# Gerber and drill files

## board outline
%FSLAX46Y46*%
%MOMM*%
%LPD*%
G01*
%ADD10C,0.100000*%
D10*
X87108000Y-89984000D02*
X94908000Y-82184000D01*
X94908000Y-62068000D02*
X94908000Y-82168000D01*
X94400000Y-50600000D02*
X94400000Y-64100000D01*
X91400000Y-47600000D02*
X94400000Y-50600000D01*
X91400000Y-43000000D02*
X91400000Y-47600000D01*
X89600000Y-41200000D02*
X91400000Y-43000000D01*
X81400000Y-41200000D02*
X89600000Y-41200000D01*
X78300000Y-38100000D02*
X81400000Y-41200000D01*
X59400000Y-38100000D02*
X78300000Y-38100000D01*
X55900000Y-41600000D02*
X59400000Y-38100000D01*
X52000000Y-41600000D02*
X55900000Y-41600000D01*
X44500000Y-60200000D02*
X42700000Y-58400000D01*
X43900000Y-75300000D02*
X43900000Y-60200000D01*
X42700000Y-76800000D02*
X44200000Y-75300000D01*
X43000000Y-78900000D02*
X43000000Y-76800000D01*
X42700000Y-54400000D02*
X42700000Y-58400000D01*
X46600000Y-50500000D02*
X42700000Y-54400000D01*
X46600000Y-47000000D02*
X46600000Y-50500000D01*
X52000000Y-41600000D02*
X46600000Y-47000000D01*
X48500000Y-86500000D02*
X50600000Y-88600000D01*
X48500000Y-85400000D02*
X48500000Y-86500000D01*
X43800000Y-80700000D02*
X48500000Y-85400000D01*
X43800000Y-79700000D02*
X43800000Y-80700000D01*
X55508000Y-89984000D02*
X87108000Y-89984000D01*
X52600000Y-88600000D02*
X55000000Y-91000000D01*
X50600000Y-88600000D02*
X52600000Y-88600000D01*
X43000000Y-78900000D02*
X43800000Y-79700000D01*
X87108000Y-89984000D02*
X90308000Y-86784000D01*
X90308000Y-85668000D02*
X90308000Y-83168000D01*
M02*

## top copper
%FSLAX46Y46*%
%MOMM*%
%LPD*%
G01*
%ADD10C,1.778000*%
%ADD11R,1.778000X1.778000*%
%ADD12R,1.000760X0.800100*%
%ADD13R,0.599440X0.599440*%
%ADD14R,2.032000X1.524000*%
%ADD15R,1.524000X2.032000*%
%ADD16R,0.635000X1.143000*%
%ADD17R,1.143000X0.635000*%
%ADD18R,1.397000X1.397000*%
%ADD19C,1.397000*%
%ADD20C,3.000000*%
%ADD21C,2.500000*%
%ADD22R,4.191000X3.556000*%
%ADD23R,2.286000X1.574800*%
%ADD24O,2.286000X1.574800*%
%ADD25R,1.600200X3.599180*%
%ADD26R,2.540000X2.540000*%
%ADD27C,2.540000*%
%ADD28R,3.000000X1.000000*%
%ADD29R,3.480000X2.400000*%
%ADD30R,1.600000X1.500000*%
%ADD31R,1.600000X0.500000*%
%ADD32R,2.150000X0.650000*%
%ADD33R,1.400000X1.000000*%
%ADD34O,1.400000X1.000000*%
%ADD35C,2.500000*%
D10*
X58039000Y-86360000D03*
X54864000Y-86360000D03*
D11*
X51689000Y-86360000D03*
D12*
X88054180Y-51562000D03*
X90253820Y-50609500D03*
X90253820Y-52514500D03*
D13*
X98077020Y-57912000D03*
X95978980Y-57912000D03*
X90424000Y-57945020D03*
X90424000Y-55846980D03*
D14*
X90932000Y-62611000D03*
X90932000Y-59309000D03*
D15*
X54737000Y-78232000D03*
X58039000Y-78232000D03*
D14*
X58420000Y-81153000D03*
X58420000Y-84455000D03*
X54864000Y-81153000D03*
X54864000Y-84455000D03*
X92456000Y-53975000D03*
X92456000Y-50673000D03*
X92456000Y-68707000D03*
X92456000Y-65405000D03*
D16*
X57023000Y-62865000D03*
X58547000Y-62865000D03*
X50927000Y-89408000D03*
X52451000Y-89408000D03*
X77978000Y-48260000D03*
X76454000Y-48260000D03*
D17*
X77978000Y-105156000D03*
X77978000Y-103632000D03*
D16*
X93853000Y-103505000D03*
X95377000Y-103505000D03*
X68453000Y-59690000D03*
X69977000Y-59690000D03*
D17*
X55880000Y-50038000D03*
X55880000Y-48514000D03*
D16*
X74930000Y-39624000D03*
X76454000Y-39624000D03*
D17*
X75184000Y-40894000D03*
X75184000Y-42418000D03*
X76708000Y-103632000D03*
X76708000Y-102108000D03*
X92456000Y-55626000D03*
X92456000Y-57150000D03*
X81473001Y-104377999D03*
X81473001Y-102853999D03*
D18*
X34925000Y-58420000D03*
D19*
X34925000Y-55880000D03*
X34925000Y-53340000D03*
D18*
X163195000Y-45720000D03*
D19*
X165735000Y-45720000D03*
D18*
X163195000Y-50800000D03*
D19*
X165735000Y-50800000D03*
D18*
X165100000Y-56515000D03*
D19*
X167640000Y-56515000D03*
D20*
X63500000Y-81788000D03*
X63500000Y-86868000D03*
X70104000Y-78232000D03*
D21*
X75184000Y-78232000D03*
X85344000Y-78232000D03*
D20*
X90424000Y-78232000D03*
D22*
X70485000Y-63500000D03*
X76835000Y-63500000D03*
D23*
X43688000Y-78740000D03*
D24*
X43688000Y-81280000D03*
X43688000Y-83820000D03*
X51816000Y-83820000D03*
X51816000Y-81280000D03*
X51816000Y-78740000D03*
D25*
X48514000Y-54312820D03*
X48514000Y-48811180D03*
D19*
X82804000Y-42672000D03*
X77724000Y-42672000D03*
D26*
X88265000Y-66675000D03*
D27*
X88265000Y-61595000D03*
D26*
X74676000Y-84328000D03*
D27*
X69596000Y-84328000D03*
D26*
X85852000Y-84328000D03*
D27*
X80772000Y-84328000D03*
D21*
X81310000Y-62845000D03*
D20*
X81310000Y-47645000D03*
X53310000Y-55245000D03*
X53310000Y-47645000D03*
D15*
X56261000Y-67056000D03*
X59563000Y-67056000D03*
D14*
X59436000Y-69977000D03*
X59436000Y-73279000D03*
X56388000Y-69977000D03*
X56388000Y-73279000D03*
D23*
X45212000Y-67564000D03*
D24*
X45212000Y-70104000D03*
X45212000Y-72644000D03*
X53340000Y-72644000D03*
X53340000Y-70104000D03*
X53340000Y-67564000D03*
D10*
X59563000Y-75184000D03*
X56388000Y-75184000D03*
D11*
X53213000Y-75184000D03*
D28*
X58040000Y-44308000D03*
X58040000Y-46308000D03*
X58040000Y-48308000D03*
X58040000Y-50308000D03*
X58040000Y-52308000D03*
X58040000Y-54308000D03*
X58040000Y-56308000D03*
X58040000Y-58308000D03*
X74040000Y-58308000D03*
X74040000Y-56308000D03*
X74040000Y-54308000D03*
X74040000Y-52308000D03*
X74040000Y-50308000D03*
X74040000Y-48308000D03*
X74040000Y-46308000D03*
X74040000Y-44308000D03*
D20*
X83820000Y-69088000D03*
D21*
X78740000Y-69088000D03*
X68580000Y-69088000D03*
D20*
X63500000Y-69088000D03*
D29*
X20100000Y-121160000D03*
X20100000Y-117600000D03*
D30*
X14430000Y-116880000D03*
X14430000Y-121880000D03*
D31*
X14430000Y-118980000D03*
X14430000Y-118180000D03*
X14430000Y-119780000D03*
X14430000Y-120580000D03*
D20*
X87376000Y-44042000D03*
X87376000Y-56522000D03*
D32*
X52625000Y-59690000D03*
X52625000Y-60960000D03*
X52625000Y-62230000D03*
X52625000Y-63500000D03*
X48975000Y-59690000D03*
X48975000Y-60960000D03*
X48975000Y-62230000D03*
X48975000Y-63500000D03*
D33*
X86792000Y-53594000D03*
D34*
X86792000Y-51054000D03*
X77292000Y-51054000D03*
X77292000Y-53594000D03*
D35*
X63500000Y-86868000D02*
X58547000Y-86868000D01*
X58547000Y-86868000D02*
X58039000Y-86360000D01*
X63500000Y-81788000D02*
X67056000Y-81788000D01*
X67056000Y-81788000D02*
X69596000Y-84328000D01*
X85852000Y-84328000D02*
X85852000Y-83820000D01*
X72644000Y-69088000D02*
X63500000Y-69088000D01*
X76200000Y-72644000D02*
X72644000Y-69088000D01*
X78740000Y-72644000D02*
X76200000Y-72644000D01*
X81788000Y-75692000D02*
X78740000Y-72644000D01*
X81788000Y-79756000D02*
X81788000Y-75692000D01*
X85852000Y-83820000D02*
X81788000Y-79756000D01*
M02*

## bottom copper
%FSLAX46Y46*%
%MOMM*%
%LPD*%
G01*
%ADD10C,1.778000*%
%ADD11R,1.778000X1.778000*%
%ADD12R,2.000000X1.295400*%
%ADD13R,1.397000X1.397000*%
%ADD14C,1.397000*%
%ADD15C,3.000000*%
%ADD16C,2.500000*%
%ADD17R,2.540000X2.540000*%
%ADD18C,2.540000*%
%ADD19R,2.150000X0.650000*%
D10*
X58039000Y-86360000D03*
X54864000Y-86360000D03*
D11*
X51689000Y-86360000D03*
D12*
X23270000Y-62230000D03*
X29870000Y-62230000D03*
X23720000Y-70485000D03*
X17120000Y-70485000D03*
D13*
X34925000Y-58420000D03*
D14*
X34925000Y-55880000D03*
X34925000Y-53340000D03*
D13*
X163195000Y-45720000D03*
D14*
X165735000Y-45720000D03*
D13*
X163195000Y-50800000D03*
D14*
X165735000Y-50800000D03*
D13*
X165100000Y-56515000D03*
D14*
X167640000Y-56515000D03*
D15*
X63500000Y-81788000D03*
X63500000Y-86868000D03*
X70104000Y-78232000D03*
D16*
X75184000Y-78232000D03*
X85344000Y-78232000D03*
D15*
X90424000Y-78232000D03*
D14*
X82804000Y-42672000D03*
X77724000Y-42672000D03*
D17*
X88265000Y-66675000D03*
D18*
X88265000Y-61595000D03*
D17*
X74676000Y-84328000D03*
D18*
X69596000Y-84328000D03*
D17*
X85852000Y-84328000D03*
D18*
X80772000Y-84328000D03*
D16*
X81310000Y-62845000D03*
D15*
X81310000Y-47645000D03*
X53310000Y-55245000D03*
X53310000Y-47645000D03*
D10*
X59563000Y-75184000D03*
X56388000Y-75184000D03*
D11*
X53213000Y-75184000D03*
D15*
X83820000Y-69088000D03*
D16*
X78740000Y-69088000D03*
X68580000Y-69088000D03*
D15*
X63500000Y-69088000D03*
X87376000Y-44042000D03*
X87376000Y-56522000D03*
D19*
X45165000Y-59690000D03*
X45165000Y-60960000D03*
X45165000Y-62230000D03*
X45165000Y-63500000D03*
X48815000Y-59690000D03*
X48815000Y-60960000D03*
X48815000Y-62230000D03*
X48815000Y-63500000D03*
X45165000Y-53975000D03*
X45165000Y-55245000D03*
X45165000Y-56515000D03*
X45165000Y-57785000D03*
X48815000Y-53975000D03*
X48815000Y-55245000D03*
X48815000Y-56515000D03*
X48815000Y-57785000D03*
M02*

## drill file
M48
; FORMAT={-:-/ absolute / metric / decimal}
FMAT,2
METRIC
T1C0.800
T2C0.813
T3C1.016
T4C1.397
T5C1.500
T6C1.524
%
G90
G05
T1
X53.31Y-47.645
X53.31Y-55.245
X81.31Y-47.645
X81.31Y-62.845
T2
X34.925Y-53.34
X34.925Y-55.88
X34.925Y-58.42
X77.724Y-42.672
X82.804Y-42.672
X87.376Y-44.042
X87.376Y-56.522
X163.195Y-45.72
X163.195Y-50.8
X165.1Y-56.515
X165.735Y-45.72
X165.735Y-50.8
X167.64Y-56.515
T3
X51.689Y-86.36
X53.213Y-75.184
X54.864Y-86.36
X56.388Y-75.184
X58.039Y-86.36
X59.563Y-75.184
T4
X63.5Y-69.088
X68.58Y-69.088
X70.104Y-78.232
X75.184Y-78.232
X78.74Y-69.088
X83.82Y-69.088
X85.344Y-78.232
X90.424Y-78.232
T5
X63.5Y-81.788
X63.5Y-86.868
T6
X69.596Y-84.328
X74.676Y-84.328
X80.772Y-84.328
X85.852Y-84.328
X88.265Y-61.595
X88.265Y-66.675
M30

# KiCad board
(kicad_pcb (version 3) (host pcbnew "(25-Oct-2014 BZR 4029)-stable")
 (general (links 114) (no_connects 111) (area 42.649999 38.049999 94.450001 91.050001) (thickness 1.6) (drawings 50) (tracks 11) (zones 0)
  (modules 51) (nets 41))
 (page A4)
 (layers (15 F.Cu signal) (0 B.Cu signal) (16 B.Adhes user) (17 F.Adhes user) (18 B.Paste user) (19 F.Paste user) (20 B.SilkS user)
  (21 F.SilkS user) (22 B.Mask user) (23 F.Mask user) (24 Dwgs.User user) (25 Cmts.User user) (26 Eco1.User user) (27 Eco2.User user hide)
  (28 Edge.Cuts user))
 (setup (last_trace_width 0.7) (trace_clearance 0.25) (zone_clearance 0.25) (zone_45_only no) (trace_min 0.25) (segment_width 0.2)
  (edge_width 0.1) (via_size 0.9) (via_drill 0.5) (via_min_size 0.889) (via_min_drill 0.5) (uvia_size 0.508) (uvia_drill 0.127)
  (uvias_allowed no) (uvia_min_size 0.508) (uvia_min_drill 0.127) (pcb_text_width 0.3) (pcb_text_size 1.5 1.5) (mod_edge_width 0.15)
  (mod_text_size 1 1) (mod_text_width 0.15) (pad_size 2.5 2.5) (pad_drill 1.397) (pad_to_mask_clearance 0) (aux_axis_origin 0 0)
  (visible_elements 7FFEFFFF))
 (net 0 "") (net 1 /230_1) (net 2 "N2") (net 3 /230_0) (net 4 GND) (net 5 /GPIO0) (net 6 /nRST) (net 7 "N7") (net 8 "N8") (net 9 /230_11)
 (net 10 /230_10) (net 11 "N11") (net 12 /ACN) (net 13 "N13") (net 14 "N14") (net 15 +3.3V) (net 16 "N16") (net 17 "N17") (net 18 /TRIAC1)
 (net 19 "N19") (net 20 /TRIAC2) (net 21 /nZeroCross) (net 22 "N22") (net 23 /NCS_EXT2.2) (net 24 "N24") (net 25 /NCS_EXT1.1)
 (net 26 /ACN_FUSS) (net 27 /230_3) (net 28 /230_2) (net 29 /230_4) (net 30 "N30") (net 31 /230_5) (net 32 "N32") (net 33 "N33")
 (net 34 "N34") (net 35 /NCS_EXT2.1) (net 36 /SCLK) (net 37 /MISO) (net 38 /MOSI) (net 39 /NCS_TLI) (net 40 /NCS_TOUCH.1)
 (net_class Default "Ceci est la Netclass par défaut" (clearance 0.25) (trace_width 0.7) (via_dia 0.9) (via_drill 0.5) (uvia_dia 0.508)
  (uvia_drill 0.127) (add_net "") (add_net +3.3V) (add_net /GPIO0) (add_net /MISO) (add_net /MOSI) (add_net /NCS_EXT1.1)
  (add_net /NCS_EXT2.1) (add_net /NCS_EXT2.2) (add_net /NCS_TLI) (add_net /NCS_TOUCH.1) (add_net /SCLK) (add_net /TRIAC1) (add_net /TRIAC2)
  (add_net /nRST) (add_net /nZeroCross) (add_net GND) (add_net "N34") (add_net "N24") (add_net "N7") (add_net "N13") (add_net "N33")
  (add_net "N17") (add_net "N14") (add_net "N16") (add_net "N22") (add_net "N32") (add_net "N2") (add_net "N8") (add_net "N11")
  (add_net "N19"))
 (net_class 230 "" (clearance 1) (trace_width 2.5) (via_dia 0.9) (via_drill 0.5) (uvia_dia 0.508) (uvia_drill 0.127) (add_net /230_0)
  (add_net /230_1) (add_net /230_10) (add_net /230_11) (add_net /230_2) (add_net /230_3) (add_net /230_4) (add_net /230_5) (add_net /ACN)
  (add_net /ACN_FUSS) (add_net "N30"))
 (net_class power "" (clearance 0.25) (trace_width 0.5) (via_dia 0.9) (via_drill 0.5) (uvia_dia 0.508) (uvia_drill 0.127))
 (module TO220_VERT (layer B.Cu) (at 54.864 86.36 90)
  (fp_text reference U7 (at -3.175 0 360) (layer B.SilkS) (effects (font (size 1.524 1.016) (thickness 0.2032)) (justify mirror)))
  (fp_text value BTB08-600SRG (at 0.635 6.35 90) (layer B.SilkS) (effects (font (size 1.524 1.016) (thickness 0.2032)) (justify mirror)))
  (pad 2 thru_hole circle (at 0 3.175 90) (size 1.778 1.778) (drill 1.016) (layers *.Cu *.Mask B.SilkS) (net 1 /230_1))
  (pad 3 thru_hole circle (at 0 0 90) (size 1.778 1.778) (drill 1.016) (layers *.Cu *.Mask B.SilkS) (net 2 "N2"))
  (pad 1 thru_hole rect (at 0 -3.175 90) (size 1.778 1.778) (drill 1.016) (layers *.Cu *.Mask B.SilkS) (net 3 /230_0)))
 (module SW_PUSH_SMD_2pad (layer B.Cu) (at 26.67 62.23)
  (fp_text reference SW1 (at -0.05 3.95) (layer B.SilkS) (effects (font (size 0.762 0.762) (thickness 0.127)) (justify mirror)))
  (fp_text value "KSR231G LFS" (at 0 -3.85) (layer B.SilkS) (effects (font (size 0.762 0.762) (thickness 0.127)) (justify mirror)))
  (pad 1 smd rect (at -3.4 0) (size 2 1.2954) (layers B.Cu B.Paste B.Mask) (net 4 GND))
  (pad 2 smd rect (at 3.2 0) (size 2 1.2954) (layers B.Cu B.Paste B.Mask) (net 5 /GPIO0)))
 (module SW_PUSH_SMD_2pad (layer B.Cu) (at 20.32 70.485 180)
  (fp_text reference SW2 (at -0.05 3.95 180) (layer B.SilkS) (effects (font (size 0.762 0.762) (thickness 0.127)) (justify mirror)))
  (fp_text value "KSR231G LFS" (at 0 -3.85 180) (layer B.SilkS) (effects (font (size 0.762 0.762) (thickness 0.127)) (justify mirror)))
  (pad 1 smd rect (at -3.4 0 180) (size 2 1.2954) (layers B.Cu B.Paste B.Mask) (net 4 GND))
  (pad 2 smd rect (at 3.2 0 180) (size 2 1.2954) (layers B.Cu B.Paste B.Mask) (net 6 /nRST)))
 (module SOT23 (layer F.Cu) (at 89.154 51.562 90)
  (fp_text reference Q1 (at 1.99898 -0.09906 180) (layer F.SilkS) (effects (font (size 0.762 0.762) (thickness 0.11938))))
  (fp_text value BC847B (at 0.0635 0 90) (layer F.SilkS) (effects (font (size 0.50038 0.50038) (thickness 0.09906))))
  (pad 3 smd rect (at 0 -1.09982 90) (size 0.8001 1.00076) (layers F.Cu F.Paste F.Mask) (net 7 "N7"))
  (pad 2 smd rect (at 0.9525 1.09982 90) (size 0.8001 1.00076) (layers F.Cu F.Paste F.Mask) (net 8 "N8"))
  (pad 1 smd rect (at -0.9525 1.09982 90) (size 0.8001 1.00076) (layers F.Cu F.Paste F.Mask) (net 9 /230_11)))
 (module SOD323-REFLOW (layer F.Cu) (at 97.028 57.912 180)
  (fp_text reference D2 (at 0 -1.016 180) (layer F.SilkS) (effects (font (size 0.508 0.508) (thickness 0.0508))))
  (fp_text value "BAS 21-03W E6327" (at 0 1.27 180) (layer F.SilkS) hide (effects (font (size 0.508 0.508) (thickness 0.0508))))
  (pad 1 smd rect (at -1.04902 0 180) (size 0.59944 0.59944) (layers F.Cu F.Paste F.Mask) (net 8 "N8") (clearance 0.09906))
  (pad 2 smd rect (at 1.04902 0 180) (size 0.59944 0.59944) (layers F.Cu F.Paste F.Mask) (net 9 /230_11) (clearance 0.09906)))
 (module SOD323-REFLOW (layer F.Cu) (at 90.424 56.896 90)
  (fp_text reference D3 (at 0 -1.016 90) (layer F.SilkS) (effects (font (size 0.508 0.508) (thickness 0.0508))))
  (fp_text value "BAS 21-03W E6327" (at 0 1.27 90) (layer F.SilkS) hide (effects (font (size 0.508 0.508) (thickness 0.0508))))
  (pad 1 smd rect (at -1.04902 0 90) (size 0.59944 0.59944) (layers F.Cu F.Paste F.Mask) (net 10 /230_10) (clearance 0.09906))
  (pad 2 smd rect (at 1.04902 0 90) (size 0.59944 0.59944) (layers F.Cu F.Paste F.Mask) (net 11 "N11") (clearance 0.09906)))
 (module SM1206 (layer F.Cu) (at 90.932 60.96 90)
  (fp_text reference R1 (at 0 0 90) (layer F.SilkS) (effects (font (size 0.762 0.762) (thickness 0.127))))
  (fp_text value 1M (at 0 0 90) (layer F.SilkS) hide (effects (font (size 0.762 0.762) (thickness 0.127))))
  (pad 1 smd rect (at -1.651 0 90) (size 1.524 2.032) (layers F.Cu F.Paste F.Mask) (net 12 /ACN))
  (pad 2 smd rect (at 1.651 0 90) (size 1.524 2.032) (layers F.Cu F.Paste F.Mask) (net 10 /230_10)))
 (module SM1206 (layer F.Cu) (at 56.388 78.232)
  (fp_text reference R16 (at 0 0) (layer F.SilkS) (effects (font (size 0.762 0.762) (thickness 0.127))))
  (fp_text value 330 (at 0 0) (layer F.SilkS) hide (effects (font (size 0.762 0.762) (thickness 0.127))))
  (pad 1 smd rect (at -1.651 0) (size 1.524 2.032) (layers F.Cu F.Paste F.Mask) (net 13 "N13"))
  (pad 2 smd rect (at 1.651 0) (size 1.524 2.032) (layers F.Cu F.Paste F.Mask) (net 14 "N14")))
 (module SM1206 (layer F.Cu) (at 58.42 82.804 270)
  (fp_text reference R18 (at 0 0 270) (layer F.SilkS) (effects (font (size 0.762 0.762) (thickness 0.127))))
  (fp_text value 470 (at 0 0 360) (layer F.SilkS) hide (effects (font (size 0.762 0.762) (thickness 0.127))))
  (pad 1 smd rect (at -1.651 0 270) (size 1.524 2.032) (layers F.Cu F.Paste F.Mask) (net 14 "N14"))
  (pad 2 smd rect (at 1.651 0 270) (size 1.524 2.032) (layers F.Cu F.Paste F.Mask) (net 1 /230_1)))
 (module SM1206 (layer F.Cu) (at 54.864 82.804 270)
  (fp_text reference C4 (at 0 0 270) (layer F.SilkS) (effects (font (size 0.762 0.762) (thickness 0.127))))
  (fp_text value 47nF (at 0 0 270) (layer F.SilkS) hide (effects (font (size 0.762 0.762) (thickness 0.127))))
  (pad 1 smd rect (at -1.651 0 270) (size 1.524 2.032) (layers F.Cu F.Paste F.Mask) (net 14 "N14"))
  (pad 2 smd rect (at 1.651 0 270) (size 1.524 2.032) (layers F.Cu F.Paste F.Mask) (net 2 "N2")))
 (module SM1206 (layer F.Cu) (at 92.456 52.324 90)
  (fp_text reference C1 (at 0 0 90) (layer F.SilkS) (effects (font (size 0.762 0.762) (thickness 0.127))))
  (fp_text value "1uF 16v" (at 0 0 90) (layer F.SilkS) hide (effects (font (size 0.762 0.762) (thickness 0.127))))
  (pad 1 smd rect (at -1.651 0 90) (size 1.524 2.032) (layers F.Cu F.Paste F.Mask) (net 11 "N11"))
  (pad 2 smd rect (at 1.651 0 90) (size 1.524 2.032) (layers F.Cu F.Paste F.Mask) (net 8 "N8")))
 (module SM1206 (layer F.Cu) (at 92.456 67.056 90)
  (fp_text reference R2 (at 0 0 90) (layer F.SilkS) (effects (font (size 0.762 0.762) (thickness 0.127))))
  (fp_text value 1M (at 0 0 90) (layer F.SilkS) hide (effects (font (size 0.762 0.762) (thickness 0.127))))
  (pad 1 smd rect (at -1.651 0 90) (size 1.524 2.032) (layers F.Cu F.Paste F.Mask) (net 3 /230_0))
  (pad 2 smd rect (at 1.651 0 90) (size 1.524 2.032) (layers F.Cu F.Paste F.Mask) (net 9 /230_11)))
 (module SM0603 (layer F.Cu) (at 57.785 62.865)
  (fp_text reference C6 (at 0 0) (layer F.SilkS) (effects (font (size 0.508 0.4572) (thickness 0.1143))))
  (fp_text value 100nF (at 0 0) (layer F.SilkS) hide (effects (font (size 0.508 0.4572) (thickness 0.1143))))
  (pad 1 smd rect (at -0.762 0) (size 0.635 1.143) (layers F.Cu F.Paste F.Mask) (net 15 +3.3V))
  (pad 2 smd rect (at 0.762 0) (size 0.635 1.143) (layers F.Cu F.Paste F.Mask) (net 4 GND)))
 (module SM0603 (layer F.Cu) (at 51.689 89.408)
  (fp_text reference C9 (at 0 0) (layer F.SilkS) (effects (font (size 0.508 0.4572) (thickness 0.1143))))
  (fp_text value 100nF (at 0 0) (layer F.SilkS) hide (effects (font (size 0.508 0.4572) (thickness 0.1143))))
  (pad 1 smd rect (at -0.762 0) (size 0.635 1.143) (layers F.Cu F.Paste F.Mask) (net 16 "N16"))
  (pad 2 smd rect (at 0.762 0) (size 0.635 1.143) (layers F.Cu F.Paste F.Mask) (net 4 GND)))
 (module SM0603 (layer F.Cu) (at 77.216 48.26 180)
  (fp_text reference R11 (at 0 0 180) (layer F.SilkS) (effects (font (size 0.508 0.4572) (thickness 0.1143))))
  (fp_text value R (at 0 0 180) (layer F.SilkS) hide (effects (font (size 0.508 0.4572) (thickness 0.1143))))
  (pad 1 smd rect (at -0.762 0 180) (size 0.635 1.143) (layers F.Cu F.Paste F.Mask) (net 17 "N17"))
  (pad 2 smd rect (at 0.762 0 180) (size 0.635 1.143) (layers F.Cu F.Paste F.Mask) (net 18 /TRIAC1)))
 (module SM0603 (layer F.Cu) (at 77.978 104.394 90)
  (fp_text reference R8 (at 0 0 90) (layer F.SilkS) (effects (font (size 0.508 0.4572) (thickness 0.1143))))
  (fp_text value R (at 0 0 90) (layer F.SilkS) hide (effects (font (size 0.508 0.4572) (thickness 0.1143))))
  (pad 1 smd rect (at -0.762 0 90) (size 0.635 1.143) (layers F.Cu F.Paste F.Mask) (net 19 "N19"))
  (pad 2 smd rect (at 0.762 0 90) (size 0.635 1.143) (layers F.Cu F.Paste F.Mask) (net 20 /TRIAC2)))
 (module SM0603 (layer F.Cu) (at 94.615 103.505)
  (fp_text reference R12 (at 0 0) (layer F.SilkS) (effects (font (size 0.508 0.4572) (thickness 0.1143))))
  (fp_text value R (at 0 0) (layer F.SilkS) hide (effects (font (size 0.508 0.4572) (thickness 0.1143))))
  (pad 1 smd rect (at -0.762 0) (size 0.635 1.143) (layers F.Cu F.Paste F.Mask) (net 15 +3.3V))
  (pad 2 smd rect (at 0.762 0) (size 0.635 1.143) (layers F.Cu F.Paste F.Mask) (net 16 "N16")))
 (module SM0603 (layer F.Cu) (at 69.215 59.69)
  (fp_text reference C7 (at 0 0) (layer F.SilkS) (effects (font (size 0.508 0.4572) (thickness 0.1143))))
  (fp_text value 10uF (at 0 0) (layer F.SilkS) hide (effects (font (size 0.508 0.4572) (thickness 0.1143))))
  (pad 1 smd rect (at -0.762 0) (size 0.635 1.143) (layers F.Cu F.Paste F.Mask) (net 16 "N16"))
  (pad 2 smd rect (at 0.762 0) (size 0.635 1.143) (layers F.Cu F.Paste F.Mask) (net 4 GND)))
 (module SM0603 (layer F.Cu) (at 55.88 49.276 90)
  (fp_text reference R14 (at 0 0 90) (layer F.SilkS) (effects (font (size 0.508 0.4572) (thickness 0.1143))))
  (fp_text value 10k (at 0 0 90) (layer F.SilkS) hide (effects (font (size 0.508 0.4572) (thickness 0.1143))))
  (pad 1 smd rect (at -0.762 0 90) (size 0.635 1.143) (layers F.Cu F.Paste F.Mask) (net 15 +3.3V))
  (pad 2 smd rect (at 0.762 0 90) (size 0.635 1.143) (layers F.Cu F.Paste F.Mask) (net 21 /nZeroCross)))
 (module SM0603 (layer F.Cu) (at 75.692 39.624)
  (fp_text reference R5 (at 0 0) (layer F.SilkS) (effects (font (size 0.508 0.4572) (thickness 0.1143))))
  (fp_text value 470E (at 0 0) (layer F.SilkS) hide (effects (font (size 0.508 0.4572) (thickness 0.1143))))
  (pad 1 smd rect (at -0.762 0) (size 0.635 1.143) (layers F.Cu F.Paste F.Mask) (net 15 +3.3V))
  (pad 2 smd rect (at 0.762 0) (size 0.635 1.143) (layers F.Cu F.Paste F.Mask) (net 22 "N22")))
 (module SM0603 (layer F.Cu) (at 75.184 41.656 270)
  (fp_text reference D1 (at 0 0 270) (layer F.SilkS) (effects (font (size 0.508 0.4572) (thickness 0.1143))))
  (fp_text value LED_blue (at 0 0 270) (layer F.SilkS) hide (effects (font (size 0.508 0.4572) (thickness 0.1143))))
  (pad 1 smd rect (at -0.762 0 270) (size 0.635 1.143) (layers F.Cu F.Paste F.Mask) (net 22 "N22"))
  (pad 2 smd rect (at 0.762 0 270) (size 0.635 1.143) (layers F.Cu F.Paste F.Mask) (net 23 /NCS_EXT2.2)))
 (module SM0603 (layer F.Cu) (at 76.708 102.87 90)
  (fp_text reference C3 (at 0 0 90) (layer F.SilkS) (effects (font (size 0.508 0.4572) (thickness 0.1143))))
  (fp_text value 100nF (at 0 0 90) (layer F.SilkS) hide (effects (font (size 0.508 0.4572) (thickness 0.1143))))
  (pad 1 smd rect (at -0.762 0 90) (size 0.635 1.143) (layers F.Cu F.Paste F.Mask) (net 15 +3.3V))
  (pad 2 smd rect (at 0.762 0 90) (size 0.635 1.143) (layers F.Cu F.Paste F.Mask) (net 4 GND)))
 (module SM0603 (layer F.Cu) (at 92.456 56.388 270)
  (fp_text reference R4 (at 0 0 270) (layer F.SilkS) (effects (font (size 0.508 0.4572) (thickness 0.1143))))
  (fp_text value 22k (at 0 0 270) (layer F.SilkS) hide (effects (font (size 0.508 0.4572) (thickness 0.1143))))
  (pad 1 smd rect (at -0.762 0 270) (size 0.635 1.143) (layers F.Cu F.Paste F.Mask) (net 11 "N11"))
  (pad 2 smd rect (at 0.762 0 270) (size 0.635 1.143) (layers F.Cu F.Paste F.Mask) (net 9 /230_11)))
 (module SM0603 (layer F.Cu) (at 81.473001 103.615999 90)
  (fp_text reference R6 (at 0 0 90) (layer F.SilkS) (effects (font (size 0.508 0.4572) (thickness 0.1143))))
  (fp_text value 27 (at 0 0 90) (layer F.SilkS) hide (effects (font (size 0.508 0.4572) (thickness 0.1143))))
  (pad 1 smd rect (at -0.762 0 90) (size 0.635 1.143) (layers F.Cu F.Paste F.Mask) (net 11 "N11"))
  (pad 2 smd rect (at 0.762 0 90) (size 0.635 1.143) (layers F.Cu F.Paste F.Mask) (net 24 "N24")))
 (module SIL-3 (layer F.Cu) (at 34.925 55.88 90)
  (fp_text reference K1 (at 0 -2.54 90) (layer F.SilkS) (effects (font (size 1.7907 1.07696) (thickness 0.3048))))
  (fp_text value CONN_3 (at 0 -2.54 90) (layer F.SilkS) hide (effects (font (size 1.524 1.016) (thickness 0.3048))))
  (pad 1 thru_hole rect (at -2.54 0 90) (size 1.397 1.397) (drill 0.8128) (layers *.Cu *.Mask F.SilkS) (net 4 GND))
  (pad 2 thru_hole circle (at 0 0 90) (size 1.397 1.397) (drill 0.8128) (layers *.Cu *.Mask F.SilkS) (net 23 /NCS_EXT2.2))
  (pad 3 thru_hole circle (at 2.54 0 90) (size 1.397 1.397) (drill 0.8128) (layers *.Cu *.Mask F.SilkS) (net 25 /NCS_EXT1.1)))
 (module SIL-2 (layer F.Cu) (at 164.465 45.72)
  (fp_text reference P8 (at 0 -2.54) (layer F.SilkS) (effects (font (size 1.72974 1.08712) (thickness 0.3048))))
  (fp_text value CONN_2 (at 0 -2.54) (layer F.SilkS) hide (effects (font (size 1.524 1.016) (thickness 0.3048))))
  (pad 1 thru_hole rect (at -1.27 0) (size 1.397 1.397) (drill 0.8128) (layers *.Cu *.Mask F.SilkS) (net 4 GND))
  (pad 2 thru_hole circle (at 1.27 0) (size 1.397 1.397) (drill 0.8128) (layers *.Cu *.Mask F.SilkS) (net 4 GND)))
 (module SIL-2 (layer F.Cu) (at 164.465 50.8)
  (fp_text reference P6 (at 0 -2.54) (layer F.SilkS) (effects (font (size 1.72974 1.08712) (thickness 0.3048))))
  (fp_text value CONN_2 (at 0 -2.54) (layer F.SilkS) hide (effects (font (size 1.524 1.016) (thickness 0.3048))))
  (pad 1 thru_hole rect (at -1.27 0) (size 1.397 1.397) (drill 0.8128) (layers *.Cu *.Mask F.SilkS) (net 4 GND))
  (pad 2 thru_hole circle (at 1.27 0) (size 1.397 1.397) (drill 0.8128) (layers *.Cu *.Mask F.SilkS) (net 4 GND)))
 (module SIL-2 (layer F.Cu) (at 166.37 56.515)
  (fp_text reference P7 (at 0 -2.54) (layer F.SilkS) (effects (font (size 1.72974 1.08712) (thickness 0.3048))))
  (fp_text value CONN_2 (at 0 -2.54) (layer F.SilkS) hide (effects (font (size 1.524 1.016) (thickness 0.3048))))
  (pad 1 thru_hole rect (at -1.27 0) (size 1.397 1.397) (drill 0.8128) (layers *.Cu *.Mask F.SilkS) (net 4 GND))
  (pad 2 thru_hole circle (at 1.27 0) (size 1.397 1.397) (drill 0.8128) (layers *.Cu *.Mask F.SilkS) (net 4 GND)))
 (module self (layer F.Cu) (at 63.5 84.328 270)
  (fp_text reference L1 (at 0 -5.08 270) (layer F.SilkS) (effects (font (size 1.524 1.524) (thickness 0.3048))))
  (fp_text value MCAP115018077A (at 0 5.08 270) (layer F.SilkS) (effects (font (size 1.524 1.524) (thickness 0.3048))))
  (pad 1 thru_hole circle (at -2.54 0 270) (size 3 3) (drill 1.5) (layers *.Cu *.Mask F.SilkS) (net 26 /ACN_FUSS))
  (pad 2 thru_hole circle (at 2.54 0 270) (size 3 3) (drill 1.5) (layers *.Cu *.Mask F.SilkS) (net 1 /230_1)))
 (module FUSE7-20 (layer F.Cu) (at 80.264 78.232)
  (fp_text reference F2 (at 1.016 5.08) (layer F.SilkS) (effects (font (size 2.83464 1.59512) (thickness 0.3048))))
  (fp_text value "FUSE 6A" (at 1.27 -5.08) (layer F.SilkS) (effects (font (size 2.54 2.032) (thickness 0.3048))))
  (pad 1 thru_hole circle (at -10.16 0) (size 3 3) (drill 1.397) (layers *.Cu *.Mask F.SilkS) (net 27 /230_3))
  (pad 1 thru_hole circle (at -5.08 0) (size 2.5 2.5) (drill 1.397) (layers *.Cu *.Mask F.SilkS) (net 27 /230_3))
  (pad 2 thru_hole circle (at 5.08 0) (size 2.5 2.5) (drill 1.397) (layers *.Cu *.Mask F.SilkS) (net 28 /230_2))
  (pad 2 thru_hole circle (at 10.16 0) (size 3 3) (drill 1.397) (layers *.Cu *.Mask F.SilkS) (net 28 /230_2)))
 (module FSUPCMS (layer F.Cu) (at 73.66 63.5 90)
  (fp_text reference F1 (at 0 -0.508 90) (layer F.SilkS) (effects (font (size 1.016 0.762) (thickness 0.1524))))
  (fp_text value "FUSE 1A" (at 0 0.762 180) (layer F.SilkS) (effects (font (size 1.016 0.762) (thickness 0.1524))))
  (pad 1 smd rect (at 0 -3.175 90) (size 3.556 4.191) (layers F.Cu F.Paste F.Mask) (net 3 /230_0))
  (pad 2 smd rect (at 0 3.175 90) (size 3.556 4.191) (layers F.Cu F.Paste F.Mask) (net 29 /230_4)))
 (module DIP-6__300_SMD (layer F.Cu) (at 47.752 81.28 270)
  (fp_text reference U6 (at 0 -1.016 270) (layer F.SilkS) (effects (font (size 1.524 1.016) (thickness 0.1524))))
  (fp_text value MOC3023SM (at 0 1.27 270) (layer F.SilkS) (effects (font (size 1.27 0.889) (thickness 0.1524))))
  (pad 1 smd rect (at -2.54 4.064 270) (size 1.5748 2.286) (layers F.Cu F.Paste F.Mask) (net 15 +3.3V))
  (pad 2 smd oval (at 0 4.064 270) (size 1.5748 2.286) (layers F.Cu F.Paste F.Mask) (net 17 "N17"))
  (pad 3 smd oval (at 2.54 4.064 270) (size 1.5748 2.286) (layers F.Cu F.Paste F.Mask))
  (pad 4 smd oval (at 2.54 -4.064 270) (size 1.5748 2.286) (layers F.Cu F.Paste F.Mask) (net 2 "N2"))
  (pad 5 smd oval (at 0 -4.064 270) (size 1.5748 2.286) (layers F.Cu F.Paste F.Mask))
  (pad 6 smd oval (at -2.54 -4.064 270) (size 1.5748 2.286) (layers F.Cu F.Paste F.Mask) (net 13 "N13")))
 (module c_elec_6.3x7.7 (layer F.Cu) (at 48.514 51.562 270)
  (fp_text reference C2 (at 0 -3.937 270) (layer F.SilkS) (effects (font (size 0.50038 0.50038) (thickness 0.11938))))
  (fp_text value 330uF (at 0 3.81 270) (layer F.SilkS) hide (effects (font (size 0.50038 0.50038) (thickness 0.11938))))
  (pad 1 smd rect (at 2.75082 0 270) (size 3.59918 1.6002) (layers F.Cu F.Paste F.Mask) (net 15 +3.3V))
  (pad 2 smd rect (at -2.75082 0 270) (size 3.59918 1.6002) (layers F.Cu F.Paste F.Mask) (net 4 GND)))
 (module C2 (layer B.Cu) (at 80.264 42.672 180)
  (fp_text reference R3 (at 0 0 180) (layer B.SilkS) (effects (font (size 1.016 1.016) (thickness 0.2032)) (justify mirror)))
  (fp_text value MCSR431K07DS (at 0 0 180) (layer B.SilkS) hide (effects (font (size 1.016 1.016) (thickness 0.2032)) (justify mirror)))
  (pad 1 thru_hole circle (at -2.54 0 180) (size 1.397 1.397) (drill 0.8128) (layers *.Cu *.Mask B.SilkS) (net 12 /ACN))
  (pad 2 thru_hole circle (at 2.54 0 180) (size 1.397 1.397) (drill 0.8128) (layers *.Cu *.Mask B.SilkS) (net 29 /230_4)))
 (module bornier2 (layer B.Cu) (at 88.265 64.135 90)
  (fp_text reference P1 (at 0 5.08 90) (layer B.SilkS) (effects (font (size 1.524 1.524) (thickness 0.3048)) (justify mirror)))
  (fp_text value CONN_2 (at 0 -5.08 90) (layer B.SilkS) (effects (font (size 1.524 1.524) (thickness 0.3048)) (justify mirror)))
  (pad 1 thru_hole rect (at -2.54 0 90) (size 2.54 2.54) (drill 1.524) (layers *.Cu *.Mask B.SilkS) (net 3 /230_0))
  (pad 2 thru_hole circle (at 2.54 0 90) (size 2.54 2.54) (drill 1.524) (layers *.Cu *.Mask B.SilkS) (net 12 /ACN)))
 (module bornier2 (layer B.Cu) (at 72.136 84.328 180)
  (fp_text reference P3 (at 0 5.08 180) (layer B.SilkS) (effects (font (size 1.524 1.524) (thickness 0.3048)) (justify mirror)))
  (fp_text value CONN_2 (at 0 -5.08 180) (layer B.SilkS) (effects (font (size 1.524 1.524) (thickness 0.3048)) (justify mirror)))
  (pad 1 thru_hole rect (at -2.54 0 180) (size 2.54 2.54) (drill 1.524) (layers *.Cu *.Mask B.SilkS) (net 27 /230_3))
  (pad 2 thru_hole circle (at 2.54 0 180) (size 2.54 2.54) (drill 1.524) (layers *.Cu *.Mask B.SilkS) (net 26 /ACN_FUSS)))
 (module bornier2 (layer B.Cu) (at 83.312 84.328 180)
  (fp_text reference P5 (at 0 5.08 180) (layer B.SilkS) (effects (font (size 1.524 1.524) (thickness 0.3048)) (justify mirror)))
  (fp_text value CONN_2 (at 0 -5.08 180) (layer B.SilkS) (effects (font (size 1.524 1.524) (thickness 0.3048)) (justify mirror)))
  (pad 1 thru_hole rect (at -2.54 0 180) (size 2.54 2.54) (drill 1.524) (layers *.Cu *.Mask B.SilkS) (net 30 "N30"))
  (pad 2 thru_hole circle (at 2.54 0 180) (size 2.54 2.54) (drill 1.524) (layers *.Cu *.Mask B.SilkS) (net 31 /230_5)))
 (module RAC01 (layer B.Cu) (at 67.31 55.245 180)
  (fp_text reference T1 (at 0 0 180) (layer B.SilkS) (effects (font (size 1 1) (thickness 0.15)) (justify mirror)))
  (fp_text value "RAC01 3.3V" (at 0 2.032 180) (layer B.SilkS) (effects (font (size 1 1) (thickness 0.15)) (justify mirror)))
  (pad 2 thru_hole circle (at -14 -7.6 180) (size 2.5 2.5) (drill 0.8) (layers *.Cu *.Mask B.SilkS) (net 29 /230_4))
  (pad 1 thru_hole circle (at -14 7.6 180) (size 3 3) (drill 0.8) (layers *.Cu *.Mask B.SilkS) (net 12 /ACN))
  (pad 4 thru_hole circle (at 14 0 180) (size 3 3) (drill 0.8) (layers *.Cu *.Mask B.SilkS) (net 15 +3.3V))
  (pad 3 thru_hole circle (at 14 7.6 180) (size 3 3) (drill 0.8) (layers *.Cu *.Mask B.SilkS) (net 4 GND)))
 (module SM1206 (layer F.Cu) (at 57.912 67.056)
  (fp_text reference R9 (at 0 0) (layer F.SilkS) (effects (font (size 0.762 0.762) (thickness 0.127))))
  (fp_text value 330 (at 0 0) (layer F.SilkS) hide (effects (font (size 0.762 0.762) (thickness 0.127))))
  (pad 1 smd rect (at -1.651 0) (size 1.524 2.032) (layers F.Cu F.Paste F.Mask) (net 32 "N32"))
  (pad 2 smd rect (at 1.651 0) (size 1.524 2.032) (layers F.Cu F.Paste F.Mask) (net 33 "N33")))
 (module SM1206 (layer F.Cu) (at 59.436 71.628 270)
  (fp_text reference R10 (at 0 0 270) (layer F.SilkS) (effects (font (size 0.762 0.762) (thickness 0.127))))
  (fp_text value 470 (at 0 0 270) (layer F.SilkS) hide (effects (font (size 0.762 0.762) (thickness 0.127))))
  (pad 1 smd rect (at -1.651 0 270) (size 1.524 2.032) (layers F.Cu F.Paste F.Mask) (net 33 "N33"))
  (pad 2 smd rect (at 1.651 0 270) (size 1.524 2.032) (layers F.Cu F.Paste F.Mask) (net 31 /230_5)))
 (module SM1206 (layer F.Cu) (at 56.388 71.628 270)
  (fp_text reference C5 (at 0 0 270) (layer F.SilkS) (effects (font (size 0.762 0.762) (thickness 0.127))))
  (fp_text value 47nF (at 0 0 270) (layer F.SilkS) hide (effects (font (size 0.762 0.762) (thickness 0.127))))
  (pad 1 smd rect (at -1.651 0 270) (size 1.524 2.032) (layers F.Cu F.Paste F.Mask) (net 33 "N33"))
  (pad 2 smd rect (at 1.651 0 270) (size 1.524 2.032) (layers F.Cu F.Paste F.Mask) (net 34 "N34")))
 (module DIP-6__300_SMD (layer F.Cu) (at 49.276 70.104 270)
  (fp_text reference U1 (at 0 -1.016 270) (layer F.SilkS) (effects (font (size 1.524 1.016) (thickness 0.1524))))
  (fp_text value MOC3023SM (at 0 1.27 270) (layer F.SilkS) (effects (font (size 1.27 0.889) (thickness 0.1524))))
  (pad 1 smd rect (at -2.54 4.064 270) (size 1.5748 2.286) (layers F.Cu F.Paste F.Mask) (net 15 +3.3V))
  (pad 2 smd oval (at 0 4.064 270) (size 1.5748 2.286) (layers F.Cu F.Paste F.Mask) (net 19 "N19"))
  (pad 3 smd oval (at 2.54 4.064 270) (size 1.5748 2.286) (layers F.Cu F.Paste F.Mask))
  (pad 4 smd oval (at 2.54 -4.064 270) (size 1.5748 2.286) (layers F.Cu F.Paste F.Mask) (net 34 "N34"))
  (pad 5 smd oval (at 0 -4.064 270) (size 1.5748 2.286) (layers F.Cu F.Paste F.Mask))
  (pad 6 smd oval (at -2.54 -4.064 270) (size 1.5748 2.286) (layers F.Cu F.Paste F.Mask) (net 32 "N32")))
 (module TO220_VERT (layer B.Cu) (at 56.388 75.184 90)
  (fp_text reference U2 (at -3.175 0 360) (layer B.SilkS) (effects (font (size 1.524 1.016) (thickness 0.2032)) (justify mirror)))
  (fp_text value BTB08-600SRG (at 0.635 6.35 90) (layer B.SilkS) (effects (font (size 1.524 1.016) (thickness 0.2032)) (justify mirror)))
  (pad 2 thru_hole circle (at 0 3.175 90) (size 1.778 1.778) (drill 1.016) (layers *.Cu *.Mask B.SilkS) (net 31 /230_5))
  (pad 3 thru_hole circle (at 0 0 90) (size 1.778 1.778) (drill 1.016) (layers *.Cu *.Mask B.SilkS) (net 34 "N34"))
  (pad 1 thru_hole rect (at 0 -3.175 90) (size 1.778 1.778) (drill 1.016) (layers *.Cu *.Mask B.SilkS) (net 3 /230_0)))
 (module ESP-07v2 (layer F.Cu) (at 66.04 51.308)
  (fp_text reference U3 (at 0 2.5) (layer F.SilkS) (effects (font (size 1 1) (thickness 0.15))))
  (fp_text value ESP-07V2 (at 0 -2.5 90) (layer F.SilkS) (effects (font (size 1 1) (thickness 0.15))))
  (pad 1 smd rect (at -8 -7) (size 3 1) (layers F.Cu F.Paste F.Mask) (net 6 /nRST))
  (pad 2 smd rect (at -8 -5) (size 3 1) (layers F.Cu F.Paste F.Mask) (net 21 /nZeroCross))
  (pad 3 smd rect (at -8 -3) (size 3 1) (layers F.Cu F.Paste F.Mask) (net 15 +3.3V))
  (pad 4 smd rect (at -8 -1) (size 3 1) (layers F.Cu F.Paste F.Mask) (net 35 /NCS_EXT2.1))
  (pad 5 smd rect (at -8 1) (size 3 1) (layers F.Cu F.Paste F.Mask) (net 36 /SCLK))
  (pad 6 smd rect (at -8 3) (size 3 1) (layers F.Cu F.Paste F.Mask) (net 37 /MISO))
  (pad 7 smd rect (at -8 5) (size 3 1) (layers F.Cu F.Paste F.Mask) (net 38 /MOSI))
  (pad 8 smd rect (at -8 7) (size 3 1) (layers F.Cu F.Paste F.Mask) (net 15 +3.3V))
  (pad 9 smd rect (at 8 7) (size 3 1) (layers F.Cu F.Paste F.Mask) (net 4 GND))
  (pad 10 smd rect (at 8 5) (size 3 1) (layers F.Cu F.Paste F.Mask) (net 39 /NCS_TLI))
  (pad 11 smd rect (at 8 3) (size 3 1) (layers F.Cu F.Paste F.Mask) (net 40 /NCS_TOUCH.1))
  (pad 12 smd rect (at 8 1) (size 3 1) (layers F.Cu F.Paste F.Mask) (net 5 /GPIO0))
  (pad 13 smd rect (at 8 -1) (size 3 1) (layers F.Cu F.Paste F.Mask) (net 20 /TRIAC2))
  (pad 14 smd rect (at 8 -3) (size 3 1) (layers F.Cu F.Paste F.Mask) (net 18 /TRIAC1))
  (pad 15 smd rect (at 8 -5) (size 3 1) (layers F.Cu F.Paste F.Mask) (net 25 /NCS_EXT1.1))
  (pad 16 smd rect (at 8 -7) (size 3 1) (layers F.Cu F.Paste F.Mask) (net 23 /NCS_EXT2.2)))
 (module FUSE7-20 (layer F.Cu) (at 73.66 69.088 180)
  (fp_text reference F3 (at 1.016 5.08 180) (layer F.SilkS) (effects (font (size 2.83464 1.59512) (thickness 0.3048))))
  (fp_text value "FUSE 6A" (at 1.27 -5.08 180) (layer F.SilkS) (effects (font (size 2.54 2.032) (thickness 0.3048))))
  (pad 1 thru_hole circle (at -10.16 0 180) (size 3 3) (drill 1.397) (layers *.Cu *.Mask F.SilkS) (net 28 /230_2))
  (pad 1 thru_hole circle (at -5.08 0 180) (size 2.5 2.5) (drill 1.397) (layers *.Cu *.Mask F.SilkS) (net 28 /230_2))
  (pad 2 thru_hole circle (at 5.08 0 180) (size 2.5 2.5) (drill 1.397) (layers *.Cu *.Mask F.SilkS) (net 30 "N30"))
  (pad 2 thru_hole circle (at 10.16 0 180) (size 3 3) (drill 1.397) (layers *.Cu *.Mask F.SilkS) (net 30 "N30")))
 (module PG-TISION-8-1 (layer F.Cu) (at 17.78 119.38 270)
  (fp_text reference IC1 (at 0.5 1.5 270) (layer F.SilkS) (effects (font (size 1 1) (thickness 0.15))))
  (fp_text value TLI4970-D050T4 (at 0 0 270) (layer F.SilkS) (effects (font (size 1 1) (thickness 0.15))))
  (pad 7 smd rect (at 1.78 -2.32 270) (size 2.4 3.48) (layers F.Cu F.Paste F.Mask) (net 12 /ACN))
  (pad 8 smd rect (at -1.78 -2.32 270) (size 2.4 3.48) (layers F.Cu F.Paste F.Mask) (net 28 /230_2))
  (pad 1 smd rect (at -2.5 3.35 270) (size 1.5 1.6) (layers F.Cu F.Paste F.Mask) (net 4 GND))
  (pad 6 smd rect (at 2.5 3.35 270) (size 1.5 1.6) (layers F.Cu F.Paste F.Mask))
  (pad 3 smd rect (at -0.4 3.35 270) (size 0.5 1.6) (layers F.Cu F.Paste F.Mask) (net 37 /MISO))
  (pad 2 smd rect (at -1.2 3.35 270) (size 0.5 1.6) (layers F.Cu F.Paste F.Mask) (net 16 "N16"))
  (pad 4 smd rect (at 0.4 3.35 270) (size 0.5 1.6) (layers F.Cu F.Paste F.Mask) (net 36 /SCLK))
  (pad 5 smd rect (at 1.2 3.35 270) (size 0.5 1.6) (layers F.Cu F.Paste F.Mask) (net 39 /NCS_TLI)))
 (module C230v (layer B.Cu) (at 87.376 50.292 270)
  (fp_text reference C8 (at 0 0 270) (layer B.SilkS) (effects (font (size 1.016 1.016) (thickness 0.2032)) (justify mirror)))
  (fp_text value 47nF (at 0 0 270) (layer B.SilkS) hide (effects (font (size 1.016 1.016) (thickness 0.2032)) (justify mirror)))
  (pad 1 thru_hole circle (at -6.25 0 270) (size 3 3) (drill 0.8128) (layers *.Cu *.Mask B.SilkS) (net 12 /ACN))
  (pad 2 thru_hole circle (at 6.23 0 270) (size 3 3) (drill 0.8128) (layers *.Cu *.Mask B.SilkS) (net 29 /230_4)))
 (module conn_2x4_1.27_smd (layer F.Cu) (at 50.8 61.595 270)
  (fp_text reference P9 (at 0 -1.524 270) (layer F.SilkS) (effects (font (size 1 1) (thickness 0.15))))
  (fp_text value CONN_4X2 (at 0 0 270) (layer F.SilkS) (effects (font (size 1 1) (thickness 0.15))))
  (pad 1 smd rect (at -1.905 -1.825 270) (size 0.65 2.15) (layers F.Cu F.Paste F.Mask) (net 4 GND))
  (pad 3 smd rect (at -0.635 -1.825 270) (size 0.65 2.15) (layers F.Cu F.Paste F.Mask))
  (pad 5 smd rect (at 0.635 -1.825 270) (size 0.65 2.15) (layers F.Cu F.Paste F.Mask) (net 40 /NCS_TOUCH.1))
  (pad 7 smd rect (at 1.905 -1.825 270) (size 0.65 2.15) (layers F.Cu F.Paste F.Mask) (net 15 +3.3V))
  (pad 2 smd rect (at -1.905 1.825 270) (size 0.65 2.15) (layers F.Cu F.Paste F.Mask) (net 4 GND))
  (pad 4 smd rect (at -0.635 1.825 270) (size 0.65 2.15) (layers F.Cu F.Paste F.Mask) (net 38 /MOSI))
  (pad 6 smd rect (at 0.635 1.825 270) (size 0.65 2.15) (layers F.Cu F.Paste F.Mask) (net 37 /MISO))
  (pad 8 smd rect (at 1.905 1.825 270) (size 0.65 2.15) (layers F.Cu F.Paste F.Mask) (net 36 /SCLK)))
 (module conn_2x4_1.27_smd (layer B.Cu) (at 46.99 61.595 270)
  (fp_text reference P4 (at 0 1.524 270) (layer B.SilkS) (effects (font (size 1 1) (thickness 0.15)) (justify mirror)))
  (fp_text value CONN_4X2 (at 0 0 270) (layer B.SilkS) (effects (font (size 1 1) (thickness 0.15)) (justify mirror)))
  (pad 1 smd rect (at -1.905 1.825 270) (size 0.65 2.15) (layers B.Cu B.Paste B.Mask) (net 4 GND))
  (pad 3 smd rect (at -0.635 1.825 270) (size 0.65 2.15) (layers B.Cu B.Paste B.Mask) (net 25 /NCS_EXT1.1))
  (pad 5 smd rect (at 0.635 1.825 270) (size 0.65 2.15) (layers B.Cu B.Paste B.Mask) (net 5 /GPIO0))
  (pad 7 smd rect (at 1.905 1.825 270) (size 0.65 2.15) (layers B.Cu B.Paste B.Mask) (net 15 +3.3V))
  (pad 2 smd rect (at -1.905 -1.825 270) (size 0.65 2.15) (layers B.Cu B.Paste B.Mask) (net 4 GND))
  (pad 4 smd rect (at -0.635 -1.825 270) (size 0.65 2.15) (layers B.Cu B.Paste B.Mask) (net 38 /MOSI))
  (pad 6 smd rect (at 0.635 -1.825 270) (size 0.65 2.15) (layers B.Cu B.Paste B.Mask) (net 37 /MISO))
  (pad 8 smd rect (at 1.905 -1.825 270) (size 0.65 2.15) (layers B.Cu B.Paste B.Mask) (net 36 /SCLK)))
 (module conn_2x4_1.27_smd (layer B.Cu) (at 46.99 55.88 270)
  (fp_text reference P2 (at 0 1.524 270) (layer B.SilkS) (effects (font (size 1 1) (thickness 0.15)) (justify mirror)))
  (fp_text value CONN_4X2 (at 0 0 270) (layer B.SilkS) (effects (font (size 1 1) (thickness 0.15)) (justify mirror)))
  (pad 1 smd rect (at -1.905 1.825 270) (size 0.65 2.15) (layers B.Cu B.Paste B.Mask) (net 4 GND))
  (pad 3 smd rect (at -0.635 1.825 270) (size 0.65 2.15) (layers B.Cu B.Paste B.Mask) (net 35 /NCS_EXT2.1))
  (pad 5 smd rect (at 0.635 1.825 270) (size 0.65 2.15) (layers B.Cu B.Paste B.Mask) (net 23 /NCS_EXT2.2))
  (pad 7 smd rect (at 1.905 1.825 270) (size 0.65 2.15) (layers B.Cu B.Paste B.Mask) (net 15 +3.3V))
  (pad 2 smd rect (at -1.905 -1.825 270) (size 0.65 2.15) (layers B.Cu B.Paste B.Mask) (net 4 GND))
  (pad 4 smd rect (at -0.635 -1.825 270) (size 0.65 2.15) (layers B.Cu B.Paste B.Mask) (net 38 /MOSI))
  (pad 6 smd rect (at 0.635 -1.825 270) (size 0.65 2.15) (layers B.Cu B.Paste B.Mask) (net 37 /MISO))
  (pad 8 smd rect (at 1.905 -1.825 270) (size 0.65 2.15) (layers B.Cu B.Paste B.Mask) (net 36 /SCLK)))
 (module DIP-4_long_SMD (layer F.Cu) (at 82.042 51.054 90)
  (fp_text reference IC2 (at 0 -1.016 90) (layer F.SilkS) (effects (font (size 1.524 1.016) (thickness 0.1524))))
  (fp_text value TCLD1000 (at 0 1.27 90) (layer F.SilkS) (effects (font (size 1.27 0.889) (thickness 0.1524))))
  (pad 1 smd rect (at -2.54 4.75 90) (size 1 1.4) (layers F.Cu F.Paste F.Mask) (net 24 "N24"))
  (pad 2 smd oval (at 0 4.75 90) (size 1 1.4) (layers F.Cu F.Paste F.Mask) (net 7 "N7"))
  (pad 3 smd oval (at 0 -4.75 90) (size 1 1.4) (layers F.Cu F.Paste F.Mask) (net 4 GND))
  (pad 4 smd oval (at -2.54 -4.75 90) (size 1 1.4) (layers F.Cu F.Paste F.Mask) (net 21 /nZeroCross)))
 (gr_line (start 87.108 89.984) (end 94.908 82.184) (angle 90) (layer Edge.Cuts) (width 0.1))
 (gr_line (start 94.908 62.068) (end 94.908 82.168) (angle 90) (layer Edge.Cuts) (width 0.1))
 (gr_line (start 94.4 50.6) (end 94.4 64.1) (angle 90) (layer Edge.Cuts) (width 0.1))
 (gr_line (start 91.4 47.6) (end 94.4 50.6) (angle 90) (layer Edge.Cuts) (width 0.1))
 (gr_line (start 91.4 43) (end 91.4 47.6) (angle 90) (layer Edge.Cuts) (width 0.1))
 (gr_line (start 89.6 41.2) (end 91.4 43) (angle 90) (layer Edge.Cuts) (width 0.1))
 (gr_line (start 81.4 41.2) (end 89.6 41.2) (angle 90) (layer Edge.Cuts) (width 0.1))
 (gr_line (start 78.3 38.1) (end 81.4 41.2) (angle 90) (layer Edge.Cuts) (width 0.1))
 (gr_line (start 59.4 38.1) (end 78.3 38.1) (angle 90) (layer Edge.Cuts) (width 0.1))
 (gr_line (start 55.9 41.6) (end 59.4 38.1) (angle 90) (layer Edge.Cuts) (width 0.1))
 (gr_line (start 52 41.6) (end 55.9 41.6) (angle 90) (layer Edge.Cuts) (width 0.1))
 (gr_line (start 44.5 60.2) (end 42.7 58.4) (angle 90) (layer Edge.Cuts) (width 0.1))
 (gr_line (start 43.9 75.3) (end 43.9 60.2) (angle 90) (layer Edge.Cuts) (width 0.1))
 (gr_line (start 42.7 76.8) (end 44.2 75.3) (angle 90) (layer Edge.Cuts) (width 0.1))
 (gr_line (start 43 78.9) (end 43 76.8) (angle 90) (layer Edge.Cuts) (width 0.1))
 (gr_line (start 42.7 54.4) (end 42.7 58.4) (angle 90) (layer Edge.Cuts) (width 0.1))
 (gr_line (start 46.6 50.5) (end 42.7 54.4) (angle 90) (layer Edge.Cuts) (width 0.1))
 (gr_line (start 46.6 47) (end 46.6 50.5) (angle 90) (layer Edge.Cuts) (width 0.1))
 (gr_line (start 52 41.6) (end 46.6 47) (angle 90) (layer Edge.Cuts) (width 0.1))
 (gr_line (start 48.5 86.5) (end 50.6 88.6) (angle 90) (layer Edge.Cuts) (width 0.1))
 (gr_line (start 48.5 85.4) (end 48.5 86.5) (angle 90) (layer Edge.Cuts) (width 0.1))
 (gr_line (start 43.8 80.7) (end 48.5 85.4) (angle 90) (layer Edge.Cuts) (width 0.1))
 (gr_line (start 43.8 79.7) (end 43.8 80.7) (angle 90) (layer Edge.Cuts) (width 0.1))
 (gr_line (start 55.508 89.984) (end 87.108 89.984) (angle 90) (layer Edge.Cuts) (width 0.1))
 (gr_line (start 52.6 88.6) (end 55 91) (angle 90) (layer Edge.Cuts) (width 0.1))
 (gr_line (start 50.6 88.6) (end 52.6 88.6) (angle 90) (layer Edge.Cuts) (width 0.1))
 (gr_line (start 43 78.9) (end 43.8 79.7) (angle 90) (layer Edge.Cuts) (width 0.1))
 (gr_line (start 87.108 89.984) (end 90.308 86.784) (angle 90) (layer Edge.Cuts) (width 0.1))
 (gr_line (start 90.308 85.668) (end 90.308 83.168) (angle 90) (layer Edge.Cuts) (width 0.1))
 (segment (start 63.5 86.868) (end 58.547 86.868) (width 2.5) (layer F.Cu) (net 1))
 (segment (start 58.547 86.868) (end 58.039 86.36) (width 2.5) (layer F.Cu) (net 1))
 (segment (start 63.5 81.788) (end 67.056 81.788) (width 2.5) (layer F.Cu) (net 26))
 (segment (start 67.056 81.788) (end 69.596 84.328) (width 2.5) (layer F.Cu) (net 26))
 (segment (start 85.852 84.328) (end 85.852 83.82) (width 2.5) (layer F.Cu) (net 30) (status C00000))
 (segment (start 72.644 69.088) (end 63.5 69.088) (width 2.5) (layer F.Cu) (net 30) (status 800000))
 (segment (start 76.2 72.644) (end 72.644 69.088) (width 2.5) (layer F.Cu) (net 30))
 (segment (start 78.74 72.644) (end 76.2 72.644) (width 2.5) (layer F.Cu) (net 30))
 (segment (start 81.788 75.692) (end 78.74 72.644) (width 2.5) (layer F.Cu) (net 30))
 (segment (start 81.788 79.756) (end 81.788 75.692) (width 2.5) (layer F.Cu) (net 30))
 (segment (start 85.852 83.82) (end 81.788 79.756) (width 2.5) (layer F.Cu) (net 30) (status 400000)))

